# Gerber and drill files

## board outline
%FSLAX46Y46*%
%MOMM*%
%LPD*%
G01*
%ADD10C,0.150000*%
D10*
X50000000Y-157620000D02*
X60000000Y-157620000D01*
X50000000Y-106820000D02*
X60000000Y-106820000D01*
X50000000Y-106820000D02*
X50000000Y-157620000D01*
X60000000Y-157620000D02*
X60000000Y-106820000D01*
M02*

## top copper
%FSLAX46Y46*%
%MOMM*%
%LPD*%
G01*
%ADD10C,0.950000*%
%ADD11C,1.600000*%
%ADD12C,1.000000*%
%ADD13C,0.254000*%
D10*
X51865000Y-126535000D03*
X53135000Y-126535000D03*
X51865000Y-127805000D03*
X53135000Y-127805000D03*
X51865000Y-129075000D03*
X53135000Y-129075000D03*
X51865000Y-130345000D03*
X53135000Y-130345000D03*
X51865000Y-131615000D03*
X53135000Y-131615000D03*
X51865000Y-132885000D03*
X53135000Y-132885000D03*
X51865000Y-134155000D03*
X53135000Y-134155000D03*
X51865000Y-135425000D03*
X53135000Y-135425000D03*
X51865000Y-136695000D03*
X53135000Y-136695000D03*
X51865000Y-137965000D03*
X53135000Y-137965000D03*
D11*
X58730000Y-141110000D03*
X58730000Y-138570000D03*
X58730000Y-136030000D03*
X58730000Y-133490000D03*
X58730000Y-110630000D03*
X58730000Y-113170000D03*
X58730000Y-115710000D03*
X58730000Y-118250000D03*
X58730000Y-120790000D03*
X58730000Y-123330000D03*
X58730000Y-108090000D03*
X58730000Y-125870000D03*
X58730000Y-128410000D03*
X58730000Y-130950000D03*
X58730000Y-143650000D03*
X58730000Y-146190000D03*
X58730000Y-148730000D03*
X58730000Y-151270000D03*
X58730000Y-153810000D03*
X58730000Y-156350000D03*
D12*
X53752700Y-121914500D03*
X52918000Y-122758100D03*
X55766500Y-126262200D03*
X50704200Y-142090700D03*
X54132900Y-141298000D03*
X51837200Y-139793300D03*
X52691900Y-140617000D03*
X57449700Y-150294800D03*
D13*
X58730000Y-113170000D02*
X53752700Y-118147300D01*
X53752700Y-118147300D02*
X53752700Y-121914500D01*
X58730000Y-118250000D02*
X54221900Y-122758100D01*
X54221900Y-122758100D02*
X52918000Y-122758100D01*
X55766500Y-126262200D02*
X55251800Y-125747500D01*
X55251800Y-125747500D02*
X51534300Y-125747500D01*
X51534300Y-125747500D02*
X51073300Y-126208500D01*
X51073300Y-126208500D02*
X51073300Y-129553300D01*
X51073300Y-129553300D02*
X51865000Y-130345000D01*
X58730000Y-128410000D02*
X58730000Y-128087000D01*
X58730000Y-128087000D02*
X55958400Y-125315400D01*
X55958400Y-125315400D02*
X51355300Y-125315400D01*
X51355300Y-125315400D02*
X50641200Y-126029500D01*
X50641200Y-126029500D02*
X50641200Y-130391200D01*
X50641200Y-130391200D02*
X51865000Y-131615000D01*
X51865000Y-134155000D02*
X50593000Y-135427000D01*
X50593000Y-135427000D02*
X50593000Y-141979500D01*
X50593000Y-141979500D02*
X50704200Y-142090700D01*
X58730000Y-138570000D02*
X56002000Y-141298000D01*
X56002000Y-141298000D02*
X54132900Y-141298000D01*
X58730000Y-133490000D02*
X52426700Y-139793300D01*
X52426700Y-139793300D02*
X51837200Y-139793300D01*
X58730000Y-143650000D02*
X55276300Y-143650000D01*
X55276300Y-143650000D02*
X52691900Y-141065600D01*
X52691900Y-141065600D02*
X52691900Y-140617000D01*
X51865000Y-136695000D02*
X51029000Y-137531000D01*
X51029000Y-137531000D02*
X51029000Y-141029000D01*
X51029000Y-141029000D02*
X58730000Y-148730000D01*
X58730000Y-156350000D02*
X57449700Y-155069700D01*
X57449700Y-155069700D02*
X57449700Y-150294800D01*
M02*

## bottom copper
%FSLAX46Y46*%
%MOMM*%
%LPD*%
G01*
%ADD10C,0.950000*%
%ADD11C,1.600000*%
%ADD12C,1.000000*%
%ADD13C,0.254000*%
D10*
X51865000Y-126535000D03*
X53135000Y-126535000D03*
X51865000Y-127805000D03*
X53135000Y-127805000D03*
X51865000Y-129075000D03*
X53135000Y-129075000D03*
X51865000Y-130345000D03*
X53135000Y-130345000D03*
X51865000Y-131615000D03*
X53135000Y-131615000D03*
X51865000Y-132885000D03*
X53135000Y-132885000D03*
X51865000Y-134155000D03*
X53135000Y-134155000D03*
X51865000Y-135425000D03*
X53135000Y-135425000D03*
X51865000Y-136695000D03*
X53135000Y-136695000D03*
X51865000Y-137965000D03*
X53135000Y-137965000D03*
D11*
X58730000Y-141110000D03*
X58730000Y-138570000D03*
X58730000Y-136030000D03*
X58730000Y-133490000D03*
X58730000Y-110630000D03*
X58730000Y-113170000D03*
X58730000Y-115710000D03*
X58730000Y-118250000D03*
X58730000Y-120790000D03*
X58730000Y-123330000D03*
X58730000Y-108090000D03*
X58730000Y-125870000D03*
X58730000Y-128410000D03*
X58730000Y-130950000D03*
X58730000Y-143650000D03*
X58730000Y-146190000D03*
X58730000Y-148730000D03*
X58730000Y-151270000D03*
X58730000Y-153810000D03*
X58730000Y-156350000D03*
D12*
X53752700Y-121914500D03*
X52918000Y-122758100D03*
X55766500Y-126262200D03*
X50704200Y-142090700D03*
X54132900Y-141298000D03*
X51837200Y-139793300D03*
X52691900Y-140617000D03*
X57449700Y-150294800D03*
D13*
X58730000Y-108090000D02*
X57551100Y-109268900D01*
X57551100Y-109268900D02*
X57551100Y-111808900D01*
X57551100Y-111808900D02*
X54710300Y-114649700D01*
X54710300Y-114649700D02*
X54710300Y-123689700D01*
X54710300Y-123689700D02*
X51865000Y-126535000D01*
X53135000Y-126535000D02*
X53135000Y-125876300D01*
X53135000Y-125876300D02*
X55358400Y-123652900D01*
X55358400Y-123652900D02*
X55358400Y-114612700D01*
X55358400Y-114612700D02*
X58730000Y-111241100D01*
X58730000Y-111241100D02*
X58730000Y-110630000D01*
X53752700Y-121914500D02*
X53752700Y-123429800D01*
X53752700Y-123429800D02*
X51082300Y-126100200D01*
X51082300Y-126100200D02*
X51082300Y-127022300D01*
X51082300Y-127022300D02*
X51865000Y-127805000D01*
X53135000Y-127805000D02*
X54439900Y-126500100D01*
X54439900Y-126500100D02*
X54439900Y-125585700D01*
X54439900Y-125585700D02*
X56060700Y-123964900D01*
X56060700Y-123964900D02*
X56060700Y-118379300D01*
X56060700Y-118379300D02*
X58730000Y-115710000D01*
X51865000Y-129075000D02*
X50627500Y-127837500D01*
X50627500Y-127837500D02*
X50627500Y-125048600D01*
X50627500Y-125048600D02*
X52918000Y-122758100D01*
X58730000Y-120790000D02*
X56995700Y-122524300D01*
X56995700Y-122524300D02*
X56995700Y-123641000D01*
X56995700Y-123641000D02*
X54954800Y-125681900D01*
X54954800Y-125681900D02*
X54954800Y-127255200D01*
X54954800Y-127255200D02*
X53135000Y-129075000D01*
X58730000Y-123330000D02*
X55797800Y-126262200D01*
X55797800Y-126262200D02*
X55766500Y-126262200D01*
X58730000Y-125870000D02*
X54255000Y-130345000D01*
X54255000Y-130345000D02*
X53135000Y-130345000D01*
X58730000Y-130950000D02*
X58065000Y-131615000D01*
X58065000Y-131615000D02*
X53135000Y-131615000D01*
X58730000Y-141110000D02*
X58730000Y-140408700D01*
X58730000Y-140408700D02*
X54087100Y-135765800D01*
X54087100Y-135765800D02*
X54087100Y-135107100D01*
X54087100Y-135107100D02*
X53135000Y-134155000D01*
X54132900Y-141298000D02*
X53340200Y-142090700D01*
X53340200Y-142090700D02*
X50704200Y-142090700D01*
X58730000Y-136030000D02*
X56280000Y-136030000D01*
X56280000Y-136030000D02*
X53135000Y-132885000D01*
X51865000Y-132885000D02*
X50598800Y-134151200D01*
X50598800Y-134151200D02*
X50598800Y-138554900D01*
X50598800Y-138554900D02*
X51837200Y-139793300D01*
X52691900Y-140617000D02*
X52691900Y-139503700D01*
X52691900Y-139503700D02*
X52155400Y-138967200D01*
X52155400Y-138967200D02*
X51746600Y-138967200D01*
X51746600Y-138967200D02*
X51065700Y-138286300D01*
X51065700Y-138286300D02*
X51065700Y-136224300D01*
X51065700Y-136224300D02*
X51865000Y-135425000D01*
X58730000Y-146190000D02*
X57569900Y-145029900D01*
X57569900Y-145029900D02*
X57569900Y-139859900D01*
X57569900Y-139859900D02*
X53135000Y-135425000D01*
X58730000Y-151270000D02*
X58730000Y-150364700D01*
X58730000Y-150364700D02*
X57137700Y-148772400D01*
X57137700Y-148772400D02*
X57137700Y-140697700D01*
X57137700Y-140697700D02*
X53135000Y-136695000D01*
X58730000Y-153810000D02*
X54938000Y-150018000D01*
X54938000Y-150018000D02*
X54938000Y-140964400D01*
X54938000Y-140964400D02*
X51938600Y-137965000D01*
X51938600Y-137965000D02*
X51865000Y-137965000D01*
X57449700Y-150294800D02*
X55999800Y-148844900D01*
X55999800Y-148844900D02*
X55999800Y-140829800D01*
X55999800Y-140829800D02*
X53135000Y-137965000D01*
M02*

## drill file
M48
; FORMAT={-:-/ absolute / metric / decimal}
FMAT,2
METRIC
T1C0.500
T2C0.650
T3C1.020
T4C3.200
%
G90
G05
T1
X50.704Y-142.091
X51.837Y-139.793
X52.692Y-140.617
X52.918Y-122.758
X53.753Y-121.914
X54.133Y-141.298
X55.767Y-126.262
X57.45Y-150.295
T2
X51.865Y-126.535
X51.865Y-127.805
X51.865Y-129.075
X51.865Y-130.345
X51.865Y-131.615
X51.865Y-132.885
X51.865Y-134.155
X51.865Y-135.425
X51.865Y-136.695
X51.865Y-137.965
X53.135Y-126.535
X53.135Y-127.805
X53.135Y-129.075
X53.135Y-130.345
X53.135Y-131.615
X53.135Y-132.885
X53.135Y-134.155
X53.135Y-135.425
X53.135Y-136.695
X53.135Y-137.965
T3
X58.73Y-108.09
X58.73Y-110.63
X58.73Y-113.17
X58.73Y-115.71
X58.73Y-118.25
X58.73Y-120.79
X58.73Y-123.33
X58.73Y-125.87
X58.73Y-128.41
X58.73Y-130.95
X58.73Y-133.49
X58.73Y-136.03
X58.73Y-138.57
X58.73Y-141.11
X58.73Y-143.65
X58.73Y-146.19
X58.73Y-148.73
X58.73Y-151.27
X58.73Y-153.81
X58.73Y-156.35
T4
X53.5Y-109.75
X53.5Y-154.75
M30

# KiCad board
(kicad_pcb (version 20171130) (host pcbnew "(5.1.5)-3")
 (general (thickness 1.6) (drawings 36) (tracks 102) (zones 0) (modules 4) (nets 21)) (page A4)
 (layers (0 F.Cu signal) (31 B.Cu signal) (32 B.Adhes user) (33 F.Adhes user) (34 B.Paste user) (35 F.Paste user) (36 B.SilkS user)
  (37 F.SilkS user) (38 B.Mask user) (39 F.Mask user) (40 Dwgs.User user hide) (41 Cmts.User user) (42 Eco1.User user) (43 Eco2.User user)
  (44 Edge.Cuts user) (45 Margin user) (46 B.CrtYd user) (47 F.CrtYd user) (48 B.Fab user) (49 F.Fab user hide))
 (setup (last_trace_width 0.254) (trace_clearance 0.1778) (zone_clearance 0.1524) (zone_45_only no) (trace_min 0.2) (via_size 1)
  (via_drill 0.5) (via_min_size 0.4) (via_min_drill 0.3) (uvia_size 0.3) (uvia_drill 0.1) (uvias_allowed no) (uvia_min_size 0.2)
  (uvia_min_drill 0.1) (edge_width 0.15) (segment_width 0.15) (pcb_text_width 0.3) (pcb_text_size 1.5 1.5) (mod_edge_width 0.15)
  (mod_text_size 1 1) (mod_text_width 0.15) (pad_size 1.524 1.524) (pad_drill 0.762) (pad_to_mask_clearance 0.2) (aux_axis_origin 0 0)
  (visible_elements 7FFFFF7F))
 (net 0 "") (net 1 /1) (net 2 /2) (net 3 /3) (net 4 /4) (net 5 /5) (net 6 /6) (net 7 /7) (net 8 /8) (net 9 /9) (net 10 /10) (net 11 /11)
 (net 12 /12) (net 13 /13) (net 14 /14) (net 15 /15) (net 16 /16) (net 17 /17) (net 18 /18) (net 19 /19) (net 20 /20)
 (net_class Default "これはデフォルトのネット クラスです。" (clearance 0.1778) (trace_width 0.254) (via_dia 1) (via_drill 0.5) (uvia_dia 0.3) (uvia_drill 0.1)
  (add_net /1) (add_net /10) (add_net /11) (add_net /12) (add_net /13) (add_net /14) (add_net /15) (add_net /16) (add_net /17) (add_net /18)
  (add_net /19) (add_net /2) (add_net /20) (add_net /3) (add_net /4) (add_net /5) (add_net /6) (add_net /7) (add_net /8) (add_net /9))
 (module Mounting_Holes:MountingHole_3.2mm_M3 (layer F.Cu) (at 53.5 154.75)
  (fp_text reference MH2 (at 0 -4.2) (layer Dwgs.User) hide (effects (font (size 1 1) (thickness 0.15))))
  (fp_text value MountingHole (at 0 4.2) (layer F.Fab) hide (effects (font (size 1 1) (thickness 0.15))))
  (pad 1 np_thru_hole circle (at 0 0) (size 3.2 3.2) (drill 3.2) (layers *.Cu *.Mask)))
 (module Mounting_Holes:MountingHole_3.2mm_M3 (layer F.Cu) (at 53.5 109.75)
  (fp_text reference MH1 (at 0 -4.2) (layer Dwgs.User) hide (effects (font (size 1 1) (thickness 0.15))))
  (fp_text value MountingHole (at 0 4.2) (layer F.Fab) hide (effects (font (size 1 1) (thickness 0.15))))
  (pad 1 np_thru_hole circle (at 0 0) (size 3.2 3.2) (drill 3.2) (layers *.Cu *.Mask)))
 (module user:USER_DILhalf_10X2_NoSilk (layer F.Cu) (at 52.5 132.25)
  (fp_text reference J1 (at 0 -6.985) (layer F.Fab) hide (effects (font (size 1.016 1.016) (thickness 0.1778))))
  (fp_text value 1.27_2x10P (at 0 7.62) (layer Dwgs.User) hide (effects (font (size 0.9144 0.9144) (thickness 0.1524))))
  (pad 1 thru_hole circle (at -0.635 -5.715) (size 0.95 0.95) (drill 0.65) (layers *.Cu *.Mask) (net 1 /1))
  (pad 2 thru_hole circle (at 0.635 -5.715) (size 0.95 0.95) (drill 0.65) (layers *.Cu *.Mask) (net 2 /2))
  (pad 3 thru_hole circle (at -0.635 -4.445) (size 0.95 0.95) (drill 0.65) (layers *.Cu *.Mask) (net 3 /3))
  (pad 4 thru_hole circle (at 0.635 -4.445) (size 0.95 0.95) (drill 0.65) (layers *.Cu *.Mask) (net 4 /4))
  (pad 5 thru_hole circle (at -0.635 -3.175) (size 0.95 0.95) (drill 0.65) (layers *.Cu *.Mask) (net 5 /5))
  (pad 6 thru_hole circle (at 0.635 -3.175) (size 0.95 0.95) (drill 0.65) (layers *.Cu *.Mask) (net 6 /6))
  (pad 7 thru_hole circle (at -0.635 -1.905) (size 0.95 0.95) (drill 0.65) (layers *.Cu *.Mask) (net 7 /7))
  (pad 8 thru_hole circle (at 0.635 -1.905) (size 0.95 0.95) (drill 0.65) (layers *.Cu *.Mask) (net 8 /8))
  (pad 9 thru_hole circle (at -0.635 -0.635) (size 0.95 0.95) (drill 0.65) (layers *.Cu *.Mask) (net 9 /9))
  (pad 10 thru_hole circle (at 0.635 -0.635) (size 0.95 0.95) (drill 0.65) (layers *.Cu *.Mask) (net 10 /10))
  (pad 11 thru_hole circle (at -0.635 0.635) (size 0.95 0.95) (drill 0.65) (layers *.Cu *.Mask) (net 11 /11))
  (pad 12 thru_hole circle (at 0.635 0.635) (size 0.95 0.95) (drill 0.65) (layers *.Cu *.Mask) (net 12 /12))
  (pad 13 thru_hole circle (at -0.635 1.905) (size 0.95 0.95) (drill 0.65) (layers *.Cu *.Mask) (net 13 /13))
  (pad 14 thru_hole circle (at 0.635 1.905) (size 0.95 0.95) (drill 0.65) (layers *.Cu *.Mask) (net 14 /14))
  (pad 15 thru_hole circle (at -0.635 3.175) (size 0.95 0.95) (drill 0.65) (layers *.Cu *.Mask) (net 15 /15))
  (pad 16 thru_hole circle (at 0.635 3.175) (size 0.95 0.95) (drill 0.65) (layers *.Cu *.Mask) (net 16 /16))
  (pad 17 thru_hole circle (at -0.635 4.445) (size 0.95 0.95) (drill 0.65) (layers *.Cu *.Mask) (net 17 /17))
  (pad 18 thru_hole circle (at 0.635 4.445) (size 0.95 0.95) (drill 0.65) (layers *.Cu *.Mask) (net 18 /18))
  (pad 19 thru_hole circle (at -0.635 5.715) (size 0.95 0.95) (drill 0.65) (layers *.Cu *.Mask) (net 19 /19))
  (pad 20 thru_hole circle (at 0.635 5.715) (size 0.95 0.95) (drill 0.65) (layers *.Cu *.Mask) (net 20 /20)))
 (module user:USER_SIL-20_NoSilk (layer F.Cu) (at 58.73 132.22 270)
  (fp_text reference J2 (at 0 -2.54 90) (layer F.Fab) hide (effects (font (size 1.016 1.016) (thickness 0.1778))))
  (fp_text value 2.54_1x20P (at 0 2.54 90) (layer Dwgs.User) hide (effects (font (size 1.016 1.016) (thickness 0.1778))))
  (pad 14 thru_hole circle (at 8.89 0 270) (size 1.6 1.6) (drill 1.02) (layers *.Cu *.Mask) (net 14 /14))
  (pad 13 thru_hole circle (at 6.35 0 270) (size 1.6 1.6) (drill 1.02) (layers *.Cu *.Mask) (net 13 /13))
  (pad 12 thru_hole circle (at 3.81 0 270) (size 1.6 1.6) (drill 1.02) (layers *.Cu *.Mask) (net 12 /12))
  (pad 11 thru_hole circle (at 1.27 0 270) (size 1.6 1.6) (drill 1.02) (layers *.Cu *.Mask) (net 11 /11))
  (pad 2 thru_hole circle (at -21.59 0 270) (size 1.6 1.6) (drill 1.02) (layers *.Cu *.Mask) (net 2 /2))
  (pad 3 thru_hole circle (at -19.05 0 270) (size 1.6 1.6) (drill 1.02) (layers *.Cu *.Mask) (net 3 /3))
  (pad 4 thru_hole circle (at -16.51 0 270) (size 1.6 1.6) (drill 1.02) (layers *.Cu *.Mask) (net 4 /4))
  (pad 5 thru_hole circle (at -13.97 0 270) (size 1.6 1.6) (drill 1.02) (layers *.Cu *.Mask) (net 5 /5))
  (pad 6 thru_hole circle (at -11.43 0 270) (size 1.6 1.6) (drill 1.02) (layers *.Cu *.Mask) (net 6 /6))
  (pad 7 thru_hole circle (at -8.89 0 270) (size 1.6 1.6) (drill 1.02) (layers *.Cu *.Mask) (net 7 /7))
  (pad 1 thru_hole circle (at -24.13 0 270) (size 1.6 1.6) (drill 1.02) (layers *.Cu *.Mask) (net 1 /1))
  (pad 8 thru_hole circle (at -6.35 0 270) (size 1.6 1.6) (drill 1.02) (layers *.Cu *.Mask) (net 8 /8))
  (pad 9 thru_hole circle (at -3.81 0 270) (size 1.6 1.6) (drill 1.02) (layers *.Cu *.Mask) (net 9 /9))
  (pad 10 thru_hole circle (at -1.27 0 270) (size 1.6 1.6) (drill 1.02) (layers *.Cu *.Mask) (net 10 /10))
  (pad 15 thru_hole circle (at 11.43 0 270) (size 1.6 1.6) (drill 1.02) (layers *.Cu *.Mask) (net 15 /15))
  (pad 16 thru_hole circle (at 13.97 0 270) (size 1.6 1.6) (drill 1.02) (layers *.Cu *.Mask) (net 16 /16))
  (pad 17 thru_hole circle (at 16.51 0 270) (size 1.6 1.6) (drill 1.02) (layers *.Cu *.Mask) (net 17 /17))
  (pad 18 thru_hole circle (at 19.05 0 270) (size 1.6 1.6) (drill 1.02) (layers *.Cu *.Mask) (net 18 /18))
  (pad 19 thru_hole circle (at 21.59 0 270) (size 1.6 1.6) (drill 1.02) (layers *.Cu *.Mask) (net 19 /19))
  (pad 20 thru_hole circle (at 24.13 0 270) (size 1.6 1.6) (drill 1.02) (layers *.Cu *.Mask) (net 20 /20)))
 (gr_line (start 50 157.62) (end 60 157.62) (angle 90) (layer Edge.Cuts) (width 0.15))
 (gr_line (start 50 106.82) (end 60 106.82) (angle 90) (layer Edge.Cuts) (width 0.15))
 (gr_line (start 50 106.82) (end 50 157.62) (angle 90) (layer Edge.Cuts) (width 0.15))
 (gr_line (start 60 157.62) (end 60 106.82) (angle 90) (layer Edge.Cuts) (width 0.15))
 (segment (start 58.73 108.09) (end 57.5511 109.2689) (width 0.254) (layer B.Cu) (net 1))
 (segment (start 57.5511 109.2689) (end 57.5511 111.8089) (width 0.254) (layer B.Cu) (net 1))
 (segment (start 57.5511 111.8089) (end 54.7103 114.6497) (width 0.254) (layer B.Cu) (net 1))
 (segment (start 54.7103 114.6497) (end 54.7103 123.6897) (width 0.254) (layer B.Cu) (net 1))
 (segment (start 54.7103 123.6897) (end 51.865 126.535) (width 0.254) (layer B.Cu) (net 1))
 (segment (start 53.135 126.535) (end 53.135 125.8763) (width 0.254) (layer B.Cu) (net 2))
 (segment (start 53.135 125.8763) (end 55.3584 123.6529) (width 0.254) (layer B.Cu) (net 2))
 (segment (start 55.3584 123.6529) (end 55.3584 114.6127) (width 0.254) (layer B.Cu) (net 2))
 (segment (start 55.3584 114.6127) (end 58.73 111.2411) (width 0.254) (layer B.Cu) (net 2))
 (segment (start 58.73 111.2411) (end 58.73 110.63) (width 0.254) (layer B.Cu) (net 2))
 (segment (start 58.73 113.17) (end 53.7527 118.1473) (width 0.254) (layer F.Cu) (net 3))
 (segment (start 53.7527 118.1473) (end 53.7527 121.9145) (width 0.254) (layer F.Cu) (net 3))
 (segment (start 53.7527 121.9145) (end 53.7527 123.4298) (width 0.254) (layer B.Cu) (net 3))
 (segment (start 53.7527 123.4298) (end 51.0823 126.1002) (width 0.254) (layer B.Cu) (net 3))
 (segment (start 51.0823 126.1002) (end 51.0823 127.0223) (width 0.254) (layer B.Cu) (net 3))
 (segment (start 51.0823 127.0223) (end 51.865 127.805) (width 0.254) (layer B.Cu) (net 3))
 (via (at 53.7527 121.9145) (size 1) (layers F.Cu B.Cu) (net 3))
 (segment (start 53.135 127.805) (end 54.4399 126.5001) (width 0.254) (layer B.Cu) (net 4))
 (segment (start 54.4399 126.5001) (end 54.4399 125.5857) (width 0.254) (layer B.Cu) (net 4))
 (segment (start 54.4399 125.5857) (end 56.0607 123.9649) (width 0.254) (layer B.Cu) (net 4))
 (segment (start 56.0607 123.9649) (end 56.0607 118.3793) (width 0.254) (layer B.Cu) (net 4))
 (segment (start 56.0607 118.3793) (end 58.73 115.71) (width 0.254) (layer B.Cu) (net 4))
 (segment (start 58.73 118.25) (end 54.2219 122.7581) (width 0.254) (layer F.Cu) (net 5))
 (segment (start 54.2219 122.7581) (end 52.918 122.7581) (width 0.254) (layer F.Cu) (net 5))
 (segment (start 51.865 129.075) (end 50.6275 127.8375) (width 0.254) (layer B.Cu) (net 5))
 (segment (start 50.6275 127.8375) (end 50.6275 125.0486) (width 0.254) (layer B.Cu) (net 5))
 (segment (start 50.6275 125.0486) (end 52.918 122.7581) (width 0.254) (layer B.Cu) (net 5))
 (via (at 52.918 122.7581) (size 1) (layers F.Cu B.Cu) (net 5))
 (segment (start 58.73 120.79) (end 56.9957 122.5243) (width 0.254) (layer B.Cu) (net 6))
 (segment (start 56.9957 122.5243) (end 56.9957 123.641) (width 0.254) (layer B.Cu) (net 6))
 (segment (start 56.9957 123.641) (end 54.9548 125.6819) (width 0.254) (layer B.Cu) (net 6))
 (segment (start 54.9548 125.6819) (end 54.9548 127.2552) (width 0.254) (layer B.Cu) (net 6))
 (segment (start 54.9548 127.2552) (end 53.135 129.075) (width 0.254) (layer B.Cu) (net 6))
 (segment (start 55.7665 126.2622) (end 55.2518 125.7475) (width 0.254) (layer F.Cu) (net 7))
 (segment (start 55.2518 125.7475) (end 51.5343 125.7475) (width 0.254) (layer F.Cu) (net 7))
 (segment (start 51.5343 125.7475) (end 51.0733 126.2085) (width 0.254) (layer F.Cu) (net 7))
 (segment (start 51.0733 126.2085) (end 51.0733 129.5533) (width 0.254) (layer F.Cu) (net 7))
 (segment (start 51.0733 129.5533) (end 51.865 130.345) (width 0.254) (layer F.Cu) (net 7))
 (segment (start 58.73 123.33) (end 55.7978 126.2622) (width 0.254) (layer B.Cu) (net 7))
 (segment (start 55.7978 126.2622) (end 55.7665 126.2622) (width 0.254) (layer B.Cu) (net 7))
 (via (at 55.7665 126.2622) (size 1) (layers F.Cu B.Cu) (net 7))
 (segment (start 58.73 125.87) (end 54.255 130.345) (width 0.254) (layer B.Cu) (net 8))
 (segment (start 54.255 130.345) (end 53.135 130.345) (width 0.254) (layer B.Cu) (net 8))
 (segment (start 58.73 128.41) (end 58.73 128.087) (width 0.254) (layer F.Cu) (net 9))
 (segment (start 58.73 128.087) (end 55.9584 125.3154) (width 0.254) (layer F.Cu) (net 9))
 (segment (start 55.9584 125.3154) (end 51.3553 125.3154) (width 0.254) (layer F.Cu) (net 9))
 (segment (start 51.3553 125.3154) (end 50.6412 126.0295) (width 0.254) (layer F.Cu) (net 9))
 (segment (start 50.6412 126.0295) (end 50.6412 130.3912) (width 0.254) (layer F.Cu) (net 9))
 (segment (start 50.6412 130.3912) (end 51.865 131.615) (width 0.254) (layer F.Cu) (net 9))
 (segment (start 58.73 130.95) (end 58.065 131.615) (width 0.254) (layer B.Cu) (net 10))
 (segment (start 58.065 131.615) (end 53.135 131.615) (width 0.254) (layer B.Cu) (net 10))
 (segment (start 58.73 141.11) (end 58.73 140.4087) (width 0.254) (layer B.Cu) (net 14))
 (segment (start 58.73 140.4087) (end 54.0871 135.7658) (width 0.254) (layer B.Cu) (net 14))
 (segment (start 54.0871 135.7658) (end 54.0871 135.1071) (width 0.254) (layer B.Cu) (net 14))
 (segment (start 54.0871 135.1071) (end 53.135 134.155) (width 0.254) (layer B.Cu) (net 14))
 (segment (start 51.865 134.155) (end 50.593 135.427) (width 0.254) (layer F.Cu) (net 13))
 (segment (start 50.593 135.427) (end 50.593 141.9795) (width 0.254) (layer F.Cu) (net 13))
 (segment (start 50.593 141.9795) (end 50.7042 142.0907) (width 0.254) (layer F.Cu) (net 13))
 (segment (start 54.1329 141.298) (end 53.3402 142.0907) (width 0.254) (layer B.Cu) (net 13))
 (segment (start 53.3402 142.0907) (end 50.7042 142.0907) (width 0.254) (layer B.Cu) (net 13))
 (segment (start 58.73 138.57) (end 56.002 141.298) (width 0.254) (layer F.Cu) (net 13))
 (segment (start 56.002 141.298) (end 54.1329 141.298) (width 0.254) (layer F.Cu) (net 13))
 (via (at 50.7042 142.0907) (size 1) (layers F.Cu B.Cu) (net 13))
 (via (at 54.1329 141.298) (size 1) (layers F.Cu B.Cu) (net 13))
 (segment (start 58.73 136.03) (end 56.28 136.03) (width 0.254) (layer B.Cu) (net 12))
 (segment (start 56.28 136.03) (end 53.135 132.885) (width 0.254) (layer B.Cu) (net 12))
 (segment (start 58.73 133.49) (end 52.4267 139.7933) (width 0.254) (layer F.Cu) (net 11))
 (segment (start 52.4267 139.7933) (end 51.8372 139.7933) (width 0.254) (layer F.Cu) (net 11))
 (segment (start 51.865 132.885) (end 50.5988 134.1512) (width 0.254) (layer B.Cu) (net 11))
 (segment (start 50.5988 134.1512) (end 50.5988 138.5549) (width 0.254) (layer B.Cu) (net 11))
 (segment (start 50.5988 138.5549) (end 51.8372 139.7933) (width 0.254) (layer B.Cu) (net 11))
 (via (at 51.8372 139.7933) (size 1) (layers F.Cu B.Cu) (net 11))
 (segment (start 52.6919 140.617) (end 52.6919 139.5037) (width 0.254) (layer B.Cu) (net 15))
 (segment (start 52.6919 139.5037) (end 52.1554 138.9672) (width 0.254) (layer B.Cu) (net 15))
 (segment (start 52.1554 138.9672) (end 51.7466 138.9672) (width 0.254) (layer B.Cu) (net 15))
 (segment (start 51.7466 138.9672) (end 51.0657 138.2863) (width 0.254) (layer B.Cu) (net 15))
 (segment (start 51.0657 138.2863) (end 51.0657 136.2243) (width 0.254) (layer B.Cu) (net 15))
 (segment (start 51.0657 136.2243) (end 51.865 135.425) (width 0.254) (layer B.Cu) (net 15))
 (segment (start 58.73 143.65) (end 55.2763 143.65) (width 0.254) (layer F.Cu) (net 15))
 (segment (start 55.2763 143.65) (end 52.6919 141.0656) (width 0.254) (layer F.Cu) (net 15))
 (segment (start 52.6919 141.0656) (end 52.6919 140.617) (width 0.254) (layer F.Cu) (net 15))
 (via (at 52.6919 140.617) (size 1) (layers F.Cu B.Cu) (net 15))
 (segment (start 58.73 146.19) (end 57.5699 145.0299) (width 0.254) (layer B.Cu) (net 16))
 (segment (start 57.5699 145.0299) (end 57.5699 139.8599) (width 0.254) (layer B.Cu) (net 16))
 (segment (start 57.5699 139.8599) (end 53.135 135.425) (width 0.254) (layer B.Cu) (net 16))
 (segment (start 51.865 136.695) (end 51.029 137.531) (width 0.254) (layer F.Cu) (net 17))
 (segment (start 51.029 137.531) (end 51.029 141.029) (width 0.254) (layer F.Cu) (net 17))
 (segment (start 51.029 141.029) (end 58.73 148.73) (width 0.254) (layer F.Cu) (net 17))
 (segment (start 58.73 151.27) (end 58.73 150.3647) (width 0.254) (layer B.Cu) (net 18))
 (segment (start 58.73 150.3647) (end 57.1377 148.7724) (width 0.254) (layer B.Cu) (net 18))
 (segment (start 57.1377 148.7724) (end 57.1377 140.6977) (width 0.254) (layer B.Cu) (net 18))
 (segment (start 57.1377 140.6977) (end 53.135 136.695) (width 0.254) (layer B.Cu) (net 18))
 (segment (start 58.73 153.81) (end 54.938 150.018) (width 0.254) (layer B.Cu) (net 19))
 (segment (start 54.938 150.018) (end 54.938 140.9644) (width 0.254) (layer B.Cu) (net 19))
 (segment (start 54.938 140.9644) (end 51.9386 137.965) (width 0.254) (layer B.Cu) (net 19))
 (segment (start 51.9386 137.965) (end 51.865 137.965) (width 0.254) (layer B.Cu) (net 19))
 (segment (start 57.4497 150.2948) (end 55.9998 148.8449) (width 0.254) (layer B.Cu) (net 20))
 (segment (start 55.9998 148.8449) (end 55.9998 140.8298) (width 0.254) (layer B.Cu) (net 20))
 (segment (start 55.9998 140.8298) (end 53.135 137.965) (width 0.254) (layer B.Cu) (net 20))
 (segment (start 58.73 156.35) (end 57.4497 155.0697) (width 0.254) (layer F.Cu) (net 20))
 (segment (start 57.4497 155.0697) (end 57.4497 150.2948) (width 0.254) (layer F.Cu) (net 20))
 (via (at 57.4497 150.2948) (size 1) (layers F.Cu B.Cu) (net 20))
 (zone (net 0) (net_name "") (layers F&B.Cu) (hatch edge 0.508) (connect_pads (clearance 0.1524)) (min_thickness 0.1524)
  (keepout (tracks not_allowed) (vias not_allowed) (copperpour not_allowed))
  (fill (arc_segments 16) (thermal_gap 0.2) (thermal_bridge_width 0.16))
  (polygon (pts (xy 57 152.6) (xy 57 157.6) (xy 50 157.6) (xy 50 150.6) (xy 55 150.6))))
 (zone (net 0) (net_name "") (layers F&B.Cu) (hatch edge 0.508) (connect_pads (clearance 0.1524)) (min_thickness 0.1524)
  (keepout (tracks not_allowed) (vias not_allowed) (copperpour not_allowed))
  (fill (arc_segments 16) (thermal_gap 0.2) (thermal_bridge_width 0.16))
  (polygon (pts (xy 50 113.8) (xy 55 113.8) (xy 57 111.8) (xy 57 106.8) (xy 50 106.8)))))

